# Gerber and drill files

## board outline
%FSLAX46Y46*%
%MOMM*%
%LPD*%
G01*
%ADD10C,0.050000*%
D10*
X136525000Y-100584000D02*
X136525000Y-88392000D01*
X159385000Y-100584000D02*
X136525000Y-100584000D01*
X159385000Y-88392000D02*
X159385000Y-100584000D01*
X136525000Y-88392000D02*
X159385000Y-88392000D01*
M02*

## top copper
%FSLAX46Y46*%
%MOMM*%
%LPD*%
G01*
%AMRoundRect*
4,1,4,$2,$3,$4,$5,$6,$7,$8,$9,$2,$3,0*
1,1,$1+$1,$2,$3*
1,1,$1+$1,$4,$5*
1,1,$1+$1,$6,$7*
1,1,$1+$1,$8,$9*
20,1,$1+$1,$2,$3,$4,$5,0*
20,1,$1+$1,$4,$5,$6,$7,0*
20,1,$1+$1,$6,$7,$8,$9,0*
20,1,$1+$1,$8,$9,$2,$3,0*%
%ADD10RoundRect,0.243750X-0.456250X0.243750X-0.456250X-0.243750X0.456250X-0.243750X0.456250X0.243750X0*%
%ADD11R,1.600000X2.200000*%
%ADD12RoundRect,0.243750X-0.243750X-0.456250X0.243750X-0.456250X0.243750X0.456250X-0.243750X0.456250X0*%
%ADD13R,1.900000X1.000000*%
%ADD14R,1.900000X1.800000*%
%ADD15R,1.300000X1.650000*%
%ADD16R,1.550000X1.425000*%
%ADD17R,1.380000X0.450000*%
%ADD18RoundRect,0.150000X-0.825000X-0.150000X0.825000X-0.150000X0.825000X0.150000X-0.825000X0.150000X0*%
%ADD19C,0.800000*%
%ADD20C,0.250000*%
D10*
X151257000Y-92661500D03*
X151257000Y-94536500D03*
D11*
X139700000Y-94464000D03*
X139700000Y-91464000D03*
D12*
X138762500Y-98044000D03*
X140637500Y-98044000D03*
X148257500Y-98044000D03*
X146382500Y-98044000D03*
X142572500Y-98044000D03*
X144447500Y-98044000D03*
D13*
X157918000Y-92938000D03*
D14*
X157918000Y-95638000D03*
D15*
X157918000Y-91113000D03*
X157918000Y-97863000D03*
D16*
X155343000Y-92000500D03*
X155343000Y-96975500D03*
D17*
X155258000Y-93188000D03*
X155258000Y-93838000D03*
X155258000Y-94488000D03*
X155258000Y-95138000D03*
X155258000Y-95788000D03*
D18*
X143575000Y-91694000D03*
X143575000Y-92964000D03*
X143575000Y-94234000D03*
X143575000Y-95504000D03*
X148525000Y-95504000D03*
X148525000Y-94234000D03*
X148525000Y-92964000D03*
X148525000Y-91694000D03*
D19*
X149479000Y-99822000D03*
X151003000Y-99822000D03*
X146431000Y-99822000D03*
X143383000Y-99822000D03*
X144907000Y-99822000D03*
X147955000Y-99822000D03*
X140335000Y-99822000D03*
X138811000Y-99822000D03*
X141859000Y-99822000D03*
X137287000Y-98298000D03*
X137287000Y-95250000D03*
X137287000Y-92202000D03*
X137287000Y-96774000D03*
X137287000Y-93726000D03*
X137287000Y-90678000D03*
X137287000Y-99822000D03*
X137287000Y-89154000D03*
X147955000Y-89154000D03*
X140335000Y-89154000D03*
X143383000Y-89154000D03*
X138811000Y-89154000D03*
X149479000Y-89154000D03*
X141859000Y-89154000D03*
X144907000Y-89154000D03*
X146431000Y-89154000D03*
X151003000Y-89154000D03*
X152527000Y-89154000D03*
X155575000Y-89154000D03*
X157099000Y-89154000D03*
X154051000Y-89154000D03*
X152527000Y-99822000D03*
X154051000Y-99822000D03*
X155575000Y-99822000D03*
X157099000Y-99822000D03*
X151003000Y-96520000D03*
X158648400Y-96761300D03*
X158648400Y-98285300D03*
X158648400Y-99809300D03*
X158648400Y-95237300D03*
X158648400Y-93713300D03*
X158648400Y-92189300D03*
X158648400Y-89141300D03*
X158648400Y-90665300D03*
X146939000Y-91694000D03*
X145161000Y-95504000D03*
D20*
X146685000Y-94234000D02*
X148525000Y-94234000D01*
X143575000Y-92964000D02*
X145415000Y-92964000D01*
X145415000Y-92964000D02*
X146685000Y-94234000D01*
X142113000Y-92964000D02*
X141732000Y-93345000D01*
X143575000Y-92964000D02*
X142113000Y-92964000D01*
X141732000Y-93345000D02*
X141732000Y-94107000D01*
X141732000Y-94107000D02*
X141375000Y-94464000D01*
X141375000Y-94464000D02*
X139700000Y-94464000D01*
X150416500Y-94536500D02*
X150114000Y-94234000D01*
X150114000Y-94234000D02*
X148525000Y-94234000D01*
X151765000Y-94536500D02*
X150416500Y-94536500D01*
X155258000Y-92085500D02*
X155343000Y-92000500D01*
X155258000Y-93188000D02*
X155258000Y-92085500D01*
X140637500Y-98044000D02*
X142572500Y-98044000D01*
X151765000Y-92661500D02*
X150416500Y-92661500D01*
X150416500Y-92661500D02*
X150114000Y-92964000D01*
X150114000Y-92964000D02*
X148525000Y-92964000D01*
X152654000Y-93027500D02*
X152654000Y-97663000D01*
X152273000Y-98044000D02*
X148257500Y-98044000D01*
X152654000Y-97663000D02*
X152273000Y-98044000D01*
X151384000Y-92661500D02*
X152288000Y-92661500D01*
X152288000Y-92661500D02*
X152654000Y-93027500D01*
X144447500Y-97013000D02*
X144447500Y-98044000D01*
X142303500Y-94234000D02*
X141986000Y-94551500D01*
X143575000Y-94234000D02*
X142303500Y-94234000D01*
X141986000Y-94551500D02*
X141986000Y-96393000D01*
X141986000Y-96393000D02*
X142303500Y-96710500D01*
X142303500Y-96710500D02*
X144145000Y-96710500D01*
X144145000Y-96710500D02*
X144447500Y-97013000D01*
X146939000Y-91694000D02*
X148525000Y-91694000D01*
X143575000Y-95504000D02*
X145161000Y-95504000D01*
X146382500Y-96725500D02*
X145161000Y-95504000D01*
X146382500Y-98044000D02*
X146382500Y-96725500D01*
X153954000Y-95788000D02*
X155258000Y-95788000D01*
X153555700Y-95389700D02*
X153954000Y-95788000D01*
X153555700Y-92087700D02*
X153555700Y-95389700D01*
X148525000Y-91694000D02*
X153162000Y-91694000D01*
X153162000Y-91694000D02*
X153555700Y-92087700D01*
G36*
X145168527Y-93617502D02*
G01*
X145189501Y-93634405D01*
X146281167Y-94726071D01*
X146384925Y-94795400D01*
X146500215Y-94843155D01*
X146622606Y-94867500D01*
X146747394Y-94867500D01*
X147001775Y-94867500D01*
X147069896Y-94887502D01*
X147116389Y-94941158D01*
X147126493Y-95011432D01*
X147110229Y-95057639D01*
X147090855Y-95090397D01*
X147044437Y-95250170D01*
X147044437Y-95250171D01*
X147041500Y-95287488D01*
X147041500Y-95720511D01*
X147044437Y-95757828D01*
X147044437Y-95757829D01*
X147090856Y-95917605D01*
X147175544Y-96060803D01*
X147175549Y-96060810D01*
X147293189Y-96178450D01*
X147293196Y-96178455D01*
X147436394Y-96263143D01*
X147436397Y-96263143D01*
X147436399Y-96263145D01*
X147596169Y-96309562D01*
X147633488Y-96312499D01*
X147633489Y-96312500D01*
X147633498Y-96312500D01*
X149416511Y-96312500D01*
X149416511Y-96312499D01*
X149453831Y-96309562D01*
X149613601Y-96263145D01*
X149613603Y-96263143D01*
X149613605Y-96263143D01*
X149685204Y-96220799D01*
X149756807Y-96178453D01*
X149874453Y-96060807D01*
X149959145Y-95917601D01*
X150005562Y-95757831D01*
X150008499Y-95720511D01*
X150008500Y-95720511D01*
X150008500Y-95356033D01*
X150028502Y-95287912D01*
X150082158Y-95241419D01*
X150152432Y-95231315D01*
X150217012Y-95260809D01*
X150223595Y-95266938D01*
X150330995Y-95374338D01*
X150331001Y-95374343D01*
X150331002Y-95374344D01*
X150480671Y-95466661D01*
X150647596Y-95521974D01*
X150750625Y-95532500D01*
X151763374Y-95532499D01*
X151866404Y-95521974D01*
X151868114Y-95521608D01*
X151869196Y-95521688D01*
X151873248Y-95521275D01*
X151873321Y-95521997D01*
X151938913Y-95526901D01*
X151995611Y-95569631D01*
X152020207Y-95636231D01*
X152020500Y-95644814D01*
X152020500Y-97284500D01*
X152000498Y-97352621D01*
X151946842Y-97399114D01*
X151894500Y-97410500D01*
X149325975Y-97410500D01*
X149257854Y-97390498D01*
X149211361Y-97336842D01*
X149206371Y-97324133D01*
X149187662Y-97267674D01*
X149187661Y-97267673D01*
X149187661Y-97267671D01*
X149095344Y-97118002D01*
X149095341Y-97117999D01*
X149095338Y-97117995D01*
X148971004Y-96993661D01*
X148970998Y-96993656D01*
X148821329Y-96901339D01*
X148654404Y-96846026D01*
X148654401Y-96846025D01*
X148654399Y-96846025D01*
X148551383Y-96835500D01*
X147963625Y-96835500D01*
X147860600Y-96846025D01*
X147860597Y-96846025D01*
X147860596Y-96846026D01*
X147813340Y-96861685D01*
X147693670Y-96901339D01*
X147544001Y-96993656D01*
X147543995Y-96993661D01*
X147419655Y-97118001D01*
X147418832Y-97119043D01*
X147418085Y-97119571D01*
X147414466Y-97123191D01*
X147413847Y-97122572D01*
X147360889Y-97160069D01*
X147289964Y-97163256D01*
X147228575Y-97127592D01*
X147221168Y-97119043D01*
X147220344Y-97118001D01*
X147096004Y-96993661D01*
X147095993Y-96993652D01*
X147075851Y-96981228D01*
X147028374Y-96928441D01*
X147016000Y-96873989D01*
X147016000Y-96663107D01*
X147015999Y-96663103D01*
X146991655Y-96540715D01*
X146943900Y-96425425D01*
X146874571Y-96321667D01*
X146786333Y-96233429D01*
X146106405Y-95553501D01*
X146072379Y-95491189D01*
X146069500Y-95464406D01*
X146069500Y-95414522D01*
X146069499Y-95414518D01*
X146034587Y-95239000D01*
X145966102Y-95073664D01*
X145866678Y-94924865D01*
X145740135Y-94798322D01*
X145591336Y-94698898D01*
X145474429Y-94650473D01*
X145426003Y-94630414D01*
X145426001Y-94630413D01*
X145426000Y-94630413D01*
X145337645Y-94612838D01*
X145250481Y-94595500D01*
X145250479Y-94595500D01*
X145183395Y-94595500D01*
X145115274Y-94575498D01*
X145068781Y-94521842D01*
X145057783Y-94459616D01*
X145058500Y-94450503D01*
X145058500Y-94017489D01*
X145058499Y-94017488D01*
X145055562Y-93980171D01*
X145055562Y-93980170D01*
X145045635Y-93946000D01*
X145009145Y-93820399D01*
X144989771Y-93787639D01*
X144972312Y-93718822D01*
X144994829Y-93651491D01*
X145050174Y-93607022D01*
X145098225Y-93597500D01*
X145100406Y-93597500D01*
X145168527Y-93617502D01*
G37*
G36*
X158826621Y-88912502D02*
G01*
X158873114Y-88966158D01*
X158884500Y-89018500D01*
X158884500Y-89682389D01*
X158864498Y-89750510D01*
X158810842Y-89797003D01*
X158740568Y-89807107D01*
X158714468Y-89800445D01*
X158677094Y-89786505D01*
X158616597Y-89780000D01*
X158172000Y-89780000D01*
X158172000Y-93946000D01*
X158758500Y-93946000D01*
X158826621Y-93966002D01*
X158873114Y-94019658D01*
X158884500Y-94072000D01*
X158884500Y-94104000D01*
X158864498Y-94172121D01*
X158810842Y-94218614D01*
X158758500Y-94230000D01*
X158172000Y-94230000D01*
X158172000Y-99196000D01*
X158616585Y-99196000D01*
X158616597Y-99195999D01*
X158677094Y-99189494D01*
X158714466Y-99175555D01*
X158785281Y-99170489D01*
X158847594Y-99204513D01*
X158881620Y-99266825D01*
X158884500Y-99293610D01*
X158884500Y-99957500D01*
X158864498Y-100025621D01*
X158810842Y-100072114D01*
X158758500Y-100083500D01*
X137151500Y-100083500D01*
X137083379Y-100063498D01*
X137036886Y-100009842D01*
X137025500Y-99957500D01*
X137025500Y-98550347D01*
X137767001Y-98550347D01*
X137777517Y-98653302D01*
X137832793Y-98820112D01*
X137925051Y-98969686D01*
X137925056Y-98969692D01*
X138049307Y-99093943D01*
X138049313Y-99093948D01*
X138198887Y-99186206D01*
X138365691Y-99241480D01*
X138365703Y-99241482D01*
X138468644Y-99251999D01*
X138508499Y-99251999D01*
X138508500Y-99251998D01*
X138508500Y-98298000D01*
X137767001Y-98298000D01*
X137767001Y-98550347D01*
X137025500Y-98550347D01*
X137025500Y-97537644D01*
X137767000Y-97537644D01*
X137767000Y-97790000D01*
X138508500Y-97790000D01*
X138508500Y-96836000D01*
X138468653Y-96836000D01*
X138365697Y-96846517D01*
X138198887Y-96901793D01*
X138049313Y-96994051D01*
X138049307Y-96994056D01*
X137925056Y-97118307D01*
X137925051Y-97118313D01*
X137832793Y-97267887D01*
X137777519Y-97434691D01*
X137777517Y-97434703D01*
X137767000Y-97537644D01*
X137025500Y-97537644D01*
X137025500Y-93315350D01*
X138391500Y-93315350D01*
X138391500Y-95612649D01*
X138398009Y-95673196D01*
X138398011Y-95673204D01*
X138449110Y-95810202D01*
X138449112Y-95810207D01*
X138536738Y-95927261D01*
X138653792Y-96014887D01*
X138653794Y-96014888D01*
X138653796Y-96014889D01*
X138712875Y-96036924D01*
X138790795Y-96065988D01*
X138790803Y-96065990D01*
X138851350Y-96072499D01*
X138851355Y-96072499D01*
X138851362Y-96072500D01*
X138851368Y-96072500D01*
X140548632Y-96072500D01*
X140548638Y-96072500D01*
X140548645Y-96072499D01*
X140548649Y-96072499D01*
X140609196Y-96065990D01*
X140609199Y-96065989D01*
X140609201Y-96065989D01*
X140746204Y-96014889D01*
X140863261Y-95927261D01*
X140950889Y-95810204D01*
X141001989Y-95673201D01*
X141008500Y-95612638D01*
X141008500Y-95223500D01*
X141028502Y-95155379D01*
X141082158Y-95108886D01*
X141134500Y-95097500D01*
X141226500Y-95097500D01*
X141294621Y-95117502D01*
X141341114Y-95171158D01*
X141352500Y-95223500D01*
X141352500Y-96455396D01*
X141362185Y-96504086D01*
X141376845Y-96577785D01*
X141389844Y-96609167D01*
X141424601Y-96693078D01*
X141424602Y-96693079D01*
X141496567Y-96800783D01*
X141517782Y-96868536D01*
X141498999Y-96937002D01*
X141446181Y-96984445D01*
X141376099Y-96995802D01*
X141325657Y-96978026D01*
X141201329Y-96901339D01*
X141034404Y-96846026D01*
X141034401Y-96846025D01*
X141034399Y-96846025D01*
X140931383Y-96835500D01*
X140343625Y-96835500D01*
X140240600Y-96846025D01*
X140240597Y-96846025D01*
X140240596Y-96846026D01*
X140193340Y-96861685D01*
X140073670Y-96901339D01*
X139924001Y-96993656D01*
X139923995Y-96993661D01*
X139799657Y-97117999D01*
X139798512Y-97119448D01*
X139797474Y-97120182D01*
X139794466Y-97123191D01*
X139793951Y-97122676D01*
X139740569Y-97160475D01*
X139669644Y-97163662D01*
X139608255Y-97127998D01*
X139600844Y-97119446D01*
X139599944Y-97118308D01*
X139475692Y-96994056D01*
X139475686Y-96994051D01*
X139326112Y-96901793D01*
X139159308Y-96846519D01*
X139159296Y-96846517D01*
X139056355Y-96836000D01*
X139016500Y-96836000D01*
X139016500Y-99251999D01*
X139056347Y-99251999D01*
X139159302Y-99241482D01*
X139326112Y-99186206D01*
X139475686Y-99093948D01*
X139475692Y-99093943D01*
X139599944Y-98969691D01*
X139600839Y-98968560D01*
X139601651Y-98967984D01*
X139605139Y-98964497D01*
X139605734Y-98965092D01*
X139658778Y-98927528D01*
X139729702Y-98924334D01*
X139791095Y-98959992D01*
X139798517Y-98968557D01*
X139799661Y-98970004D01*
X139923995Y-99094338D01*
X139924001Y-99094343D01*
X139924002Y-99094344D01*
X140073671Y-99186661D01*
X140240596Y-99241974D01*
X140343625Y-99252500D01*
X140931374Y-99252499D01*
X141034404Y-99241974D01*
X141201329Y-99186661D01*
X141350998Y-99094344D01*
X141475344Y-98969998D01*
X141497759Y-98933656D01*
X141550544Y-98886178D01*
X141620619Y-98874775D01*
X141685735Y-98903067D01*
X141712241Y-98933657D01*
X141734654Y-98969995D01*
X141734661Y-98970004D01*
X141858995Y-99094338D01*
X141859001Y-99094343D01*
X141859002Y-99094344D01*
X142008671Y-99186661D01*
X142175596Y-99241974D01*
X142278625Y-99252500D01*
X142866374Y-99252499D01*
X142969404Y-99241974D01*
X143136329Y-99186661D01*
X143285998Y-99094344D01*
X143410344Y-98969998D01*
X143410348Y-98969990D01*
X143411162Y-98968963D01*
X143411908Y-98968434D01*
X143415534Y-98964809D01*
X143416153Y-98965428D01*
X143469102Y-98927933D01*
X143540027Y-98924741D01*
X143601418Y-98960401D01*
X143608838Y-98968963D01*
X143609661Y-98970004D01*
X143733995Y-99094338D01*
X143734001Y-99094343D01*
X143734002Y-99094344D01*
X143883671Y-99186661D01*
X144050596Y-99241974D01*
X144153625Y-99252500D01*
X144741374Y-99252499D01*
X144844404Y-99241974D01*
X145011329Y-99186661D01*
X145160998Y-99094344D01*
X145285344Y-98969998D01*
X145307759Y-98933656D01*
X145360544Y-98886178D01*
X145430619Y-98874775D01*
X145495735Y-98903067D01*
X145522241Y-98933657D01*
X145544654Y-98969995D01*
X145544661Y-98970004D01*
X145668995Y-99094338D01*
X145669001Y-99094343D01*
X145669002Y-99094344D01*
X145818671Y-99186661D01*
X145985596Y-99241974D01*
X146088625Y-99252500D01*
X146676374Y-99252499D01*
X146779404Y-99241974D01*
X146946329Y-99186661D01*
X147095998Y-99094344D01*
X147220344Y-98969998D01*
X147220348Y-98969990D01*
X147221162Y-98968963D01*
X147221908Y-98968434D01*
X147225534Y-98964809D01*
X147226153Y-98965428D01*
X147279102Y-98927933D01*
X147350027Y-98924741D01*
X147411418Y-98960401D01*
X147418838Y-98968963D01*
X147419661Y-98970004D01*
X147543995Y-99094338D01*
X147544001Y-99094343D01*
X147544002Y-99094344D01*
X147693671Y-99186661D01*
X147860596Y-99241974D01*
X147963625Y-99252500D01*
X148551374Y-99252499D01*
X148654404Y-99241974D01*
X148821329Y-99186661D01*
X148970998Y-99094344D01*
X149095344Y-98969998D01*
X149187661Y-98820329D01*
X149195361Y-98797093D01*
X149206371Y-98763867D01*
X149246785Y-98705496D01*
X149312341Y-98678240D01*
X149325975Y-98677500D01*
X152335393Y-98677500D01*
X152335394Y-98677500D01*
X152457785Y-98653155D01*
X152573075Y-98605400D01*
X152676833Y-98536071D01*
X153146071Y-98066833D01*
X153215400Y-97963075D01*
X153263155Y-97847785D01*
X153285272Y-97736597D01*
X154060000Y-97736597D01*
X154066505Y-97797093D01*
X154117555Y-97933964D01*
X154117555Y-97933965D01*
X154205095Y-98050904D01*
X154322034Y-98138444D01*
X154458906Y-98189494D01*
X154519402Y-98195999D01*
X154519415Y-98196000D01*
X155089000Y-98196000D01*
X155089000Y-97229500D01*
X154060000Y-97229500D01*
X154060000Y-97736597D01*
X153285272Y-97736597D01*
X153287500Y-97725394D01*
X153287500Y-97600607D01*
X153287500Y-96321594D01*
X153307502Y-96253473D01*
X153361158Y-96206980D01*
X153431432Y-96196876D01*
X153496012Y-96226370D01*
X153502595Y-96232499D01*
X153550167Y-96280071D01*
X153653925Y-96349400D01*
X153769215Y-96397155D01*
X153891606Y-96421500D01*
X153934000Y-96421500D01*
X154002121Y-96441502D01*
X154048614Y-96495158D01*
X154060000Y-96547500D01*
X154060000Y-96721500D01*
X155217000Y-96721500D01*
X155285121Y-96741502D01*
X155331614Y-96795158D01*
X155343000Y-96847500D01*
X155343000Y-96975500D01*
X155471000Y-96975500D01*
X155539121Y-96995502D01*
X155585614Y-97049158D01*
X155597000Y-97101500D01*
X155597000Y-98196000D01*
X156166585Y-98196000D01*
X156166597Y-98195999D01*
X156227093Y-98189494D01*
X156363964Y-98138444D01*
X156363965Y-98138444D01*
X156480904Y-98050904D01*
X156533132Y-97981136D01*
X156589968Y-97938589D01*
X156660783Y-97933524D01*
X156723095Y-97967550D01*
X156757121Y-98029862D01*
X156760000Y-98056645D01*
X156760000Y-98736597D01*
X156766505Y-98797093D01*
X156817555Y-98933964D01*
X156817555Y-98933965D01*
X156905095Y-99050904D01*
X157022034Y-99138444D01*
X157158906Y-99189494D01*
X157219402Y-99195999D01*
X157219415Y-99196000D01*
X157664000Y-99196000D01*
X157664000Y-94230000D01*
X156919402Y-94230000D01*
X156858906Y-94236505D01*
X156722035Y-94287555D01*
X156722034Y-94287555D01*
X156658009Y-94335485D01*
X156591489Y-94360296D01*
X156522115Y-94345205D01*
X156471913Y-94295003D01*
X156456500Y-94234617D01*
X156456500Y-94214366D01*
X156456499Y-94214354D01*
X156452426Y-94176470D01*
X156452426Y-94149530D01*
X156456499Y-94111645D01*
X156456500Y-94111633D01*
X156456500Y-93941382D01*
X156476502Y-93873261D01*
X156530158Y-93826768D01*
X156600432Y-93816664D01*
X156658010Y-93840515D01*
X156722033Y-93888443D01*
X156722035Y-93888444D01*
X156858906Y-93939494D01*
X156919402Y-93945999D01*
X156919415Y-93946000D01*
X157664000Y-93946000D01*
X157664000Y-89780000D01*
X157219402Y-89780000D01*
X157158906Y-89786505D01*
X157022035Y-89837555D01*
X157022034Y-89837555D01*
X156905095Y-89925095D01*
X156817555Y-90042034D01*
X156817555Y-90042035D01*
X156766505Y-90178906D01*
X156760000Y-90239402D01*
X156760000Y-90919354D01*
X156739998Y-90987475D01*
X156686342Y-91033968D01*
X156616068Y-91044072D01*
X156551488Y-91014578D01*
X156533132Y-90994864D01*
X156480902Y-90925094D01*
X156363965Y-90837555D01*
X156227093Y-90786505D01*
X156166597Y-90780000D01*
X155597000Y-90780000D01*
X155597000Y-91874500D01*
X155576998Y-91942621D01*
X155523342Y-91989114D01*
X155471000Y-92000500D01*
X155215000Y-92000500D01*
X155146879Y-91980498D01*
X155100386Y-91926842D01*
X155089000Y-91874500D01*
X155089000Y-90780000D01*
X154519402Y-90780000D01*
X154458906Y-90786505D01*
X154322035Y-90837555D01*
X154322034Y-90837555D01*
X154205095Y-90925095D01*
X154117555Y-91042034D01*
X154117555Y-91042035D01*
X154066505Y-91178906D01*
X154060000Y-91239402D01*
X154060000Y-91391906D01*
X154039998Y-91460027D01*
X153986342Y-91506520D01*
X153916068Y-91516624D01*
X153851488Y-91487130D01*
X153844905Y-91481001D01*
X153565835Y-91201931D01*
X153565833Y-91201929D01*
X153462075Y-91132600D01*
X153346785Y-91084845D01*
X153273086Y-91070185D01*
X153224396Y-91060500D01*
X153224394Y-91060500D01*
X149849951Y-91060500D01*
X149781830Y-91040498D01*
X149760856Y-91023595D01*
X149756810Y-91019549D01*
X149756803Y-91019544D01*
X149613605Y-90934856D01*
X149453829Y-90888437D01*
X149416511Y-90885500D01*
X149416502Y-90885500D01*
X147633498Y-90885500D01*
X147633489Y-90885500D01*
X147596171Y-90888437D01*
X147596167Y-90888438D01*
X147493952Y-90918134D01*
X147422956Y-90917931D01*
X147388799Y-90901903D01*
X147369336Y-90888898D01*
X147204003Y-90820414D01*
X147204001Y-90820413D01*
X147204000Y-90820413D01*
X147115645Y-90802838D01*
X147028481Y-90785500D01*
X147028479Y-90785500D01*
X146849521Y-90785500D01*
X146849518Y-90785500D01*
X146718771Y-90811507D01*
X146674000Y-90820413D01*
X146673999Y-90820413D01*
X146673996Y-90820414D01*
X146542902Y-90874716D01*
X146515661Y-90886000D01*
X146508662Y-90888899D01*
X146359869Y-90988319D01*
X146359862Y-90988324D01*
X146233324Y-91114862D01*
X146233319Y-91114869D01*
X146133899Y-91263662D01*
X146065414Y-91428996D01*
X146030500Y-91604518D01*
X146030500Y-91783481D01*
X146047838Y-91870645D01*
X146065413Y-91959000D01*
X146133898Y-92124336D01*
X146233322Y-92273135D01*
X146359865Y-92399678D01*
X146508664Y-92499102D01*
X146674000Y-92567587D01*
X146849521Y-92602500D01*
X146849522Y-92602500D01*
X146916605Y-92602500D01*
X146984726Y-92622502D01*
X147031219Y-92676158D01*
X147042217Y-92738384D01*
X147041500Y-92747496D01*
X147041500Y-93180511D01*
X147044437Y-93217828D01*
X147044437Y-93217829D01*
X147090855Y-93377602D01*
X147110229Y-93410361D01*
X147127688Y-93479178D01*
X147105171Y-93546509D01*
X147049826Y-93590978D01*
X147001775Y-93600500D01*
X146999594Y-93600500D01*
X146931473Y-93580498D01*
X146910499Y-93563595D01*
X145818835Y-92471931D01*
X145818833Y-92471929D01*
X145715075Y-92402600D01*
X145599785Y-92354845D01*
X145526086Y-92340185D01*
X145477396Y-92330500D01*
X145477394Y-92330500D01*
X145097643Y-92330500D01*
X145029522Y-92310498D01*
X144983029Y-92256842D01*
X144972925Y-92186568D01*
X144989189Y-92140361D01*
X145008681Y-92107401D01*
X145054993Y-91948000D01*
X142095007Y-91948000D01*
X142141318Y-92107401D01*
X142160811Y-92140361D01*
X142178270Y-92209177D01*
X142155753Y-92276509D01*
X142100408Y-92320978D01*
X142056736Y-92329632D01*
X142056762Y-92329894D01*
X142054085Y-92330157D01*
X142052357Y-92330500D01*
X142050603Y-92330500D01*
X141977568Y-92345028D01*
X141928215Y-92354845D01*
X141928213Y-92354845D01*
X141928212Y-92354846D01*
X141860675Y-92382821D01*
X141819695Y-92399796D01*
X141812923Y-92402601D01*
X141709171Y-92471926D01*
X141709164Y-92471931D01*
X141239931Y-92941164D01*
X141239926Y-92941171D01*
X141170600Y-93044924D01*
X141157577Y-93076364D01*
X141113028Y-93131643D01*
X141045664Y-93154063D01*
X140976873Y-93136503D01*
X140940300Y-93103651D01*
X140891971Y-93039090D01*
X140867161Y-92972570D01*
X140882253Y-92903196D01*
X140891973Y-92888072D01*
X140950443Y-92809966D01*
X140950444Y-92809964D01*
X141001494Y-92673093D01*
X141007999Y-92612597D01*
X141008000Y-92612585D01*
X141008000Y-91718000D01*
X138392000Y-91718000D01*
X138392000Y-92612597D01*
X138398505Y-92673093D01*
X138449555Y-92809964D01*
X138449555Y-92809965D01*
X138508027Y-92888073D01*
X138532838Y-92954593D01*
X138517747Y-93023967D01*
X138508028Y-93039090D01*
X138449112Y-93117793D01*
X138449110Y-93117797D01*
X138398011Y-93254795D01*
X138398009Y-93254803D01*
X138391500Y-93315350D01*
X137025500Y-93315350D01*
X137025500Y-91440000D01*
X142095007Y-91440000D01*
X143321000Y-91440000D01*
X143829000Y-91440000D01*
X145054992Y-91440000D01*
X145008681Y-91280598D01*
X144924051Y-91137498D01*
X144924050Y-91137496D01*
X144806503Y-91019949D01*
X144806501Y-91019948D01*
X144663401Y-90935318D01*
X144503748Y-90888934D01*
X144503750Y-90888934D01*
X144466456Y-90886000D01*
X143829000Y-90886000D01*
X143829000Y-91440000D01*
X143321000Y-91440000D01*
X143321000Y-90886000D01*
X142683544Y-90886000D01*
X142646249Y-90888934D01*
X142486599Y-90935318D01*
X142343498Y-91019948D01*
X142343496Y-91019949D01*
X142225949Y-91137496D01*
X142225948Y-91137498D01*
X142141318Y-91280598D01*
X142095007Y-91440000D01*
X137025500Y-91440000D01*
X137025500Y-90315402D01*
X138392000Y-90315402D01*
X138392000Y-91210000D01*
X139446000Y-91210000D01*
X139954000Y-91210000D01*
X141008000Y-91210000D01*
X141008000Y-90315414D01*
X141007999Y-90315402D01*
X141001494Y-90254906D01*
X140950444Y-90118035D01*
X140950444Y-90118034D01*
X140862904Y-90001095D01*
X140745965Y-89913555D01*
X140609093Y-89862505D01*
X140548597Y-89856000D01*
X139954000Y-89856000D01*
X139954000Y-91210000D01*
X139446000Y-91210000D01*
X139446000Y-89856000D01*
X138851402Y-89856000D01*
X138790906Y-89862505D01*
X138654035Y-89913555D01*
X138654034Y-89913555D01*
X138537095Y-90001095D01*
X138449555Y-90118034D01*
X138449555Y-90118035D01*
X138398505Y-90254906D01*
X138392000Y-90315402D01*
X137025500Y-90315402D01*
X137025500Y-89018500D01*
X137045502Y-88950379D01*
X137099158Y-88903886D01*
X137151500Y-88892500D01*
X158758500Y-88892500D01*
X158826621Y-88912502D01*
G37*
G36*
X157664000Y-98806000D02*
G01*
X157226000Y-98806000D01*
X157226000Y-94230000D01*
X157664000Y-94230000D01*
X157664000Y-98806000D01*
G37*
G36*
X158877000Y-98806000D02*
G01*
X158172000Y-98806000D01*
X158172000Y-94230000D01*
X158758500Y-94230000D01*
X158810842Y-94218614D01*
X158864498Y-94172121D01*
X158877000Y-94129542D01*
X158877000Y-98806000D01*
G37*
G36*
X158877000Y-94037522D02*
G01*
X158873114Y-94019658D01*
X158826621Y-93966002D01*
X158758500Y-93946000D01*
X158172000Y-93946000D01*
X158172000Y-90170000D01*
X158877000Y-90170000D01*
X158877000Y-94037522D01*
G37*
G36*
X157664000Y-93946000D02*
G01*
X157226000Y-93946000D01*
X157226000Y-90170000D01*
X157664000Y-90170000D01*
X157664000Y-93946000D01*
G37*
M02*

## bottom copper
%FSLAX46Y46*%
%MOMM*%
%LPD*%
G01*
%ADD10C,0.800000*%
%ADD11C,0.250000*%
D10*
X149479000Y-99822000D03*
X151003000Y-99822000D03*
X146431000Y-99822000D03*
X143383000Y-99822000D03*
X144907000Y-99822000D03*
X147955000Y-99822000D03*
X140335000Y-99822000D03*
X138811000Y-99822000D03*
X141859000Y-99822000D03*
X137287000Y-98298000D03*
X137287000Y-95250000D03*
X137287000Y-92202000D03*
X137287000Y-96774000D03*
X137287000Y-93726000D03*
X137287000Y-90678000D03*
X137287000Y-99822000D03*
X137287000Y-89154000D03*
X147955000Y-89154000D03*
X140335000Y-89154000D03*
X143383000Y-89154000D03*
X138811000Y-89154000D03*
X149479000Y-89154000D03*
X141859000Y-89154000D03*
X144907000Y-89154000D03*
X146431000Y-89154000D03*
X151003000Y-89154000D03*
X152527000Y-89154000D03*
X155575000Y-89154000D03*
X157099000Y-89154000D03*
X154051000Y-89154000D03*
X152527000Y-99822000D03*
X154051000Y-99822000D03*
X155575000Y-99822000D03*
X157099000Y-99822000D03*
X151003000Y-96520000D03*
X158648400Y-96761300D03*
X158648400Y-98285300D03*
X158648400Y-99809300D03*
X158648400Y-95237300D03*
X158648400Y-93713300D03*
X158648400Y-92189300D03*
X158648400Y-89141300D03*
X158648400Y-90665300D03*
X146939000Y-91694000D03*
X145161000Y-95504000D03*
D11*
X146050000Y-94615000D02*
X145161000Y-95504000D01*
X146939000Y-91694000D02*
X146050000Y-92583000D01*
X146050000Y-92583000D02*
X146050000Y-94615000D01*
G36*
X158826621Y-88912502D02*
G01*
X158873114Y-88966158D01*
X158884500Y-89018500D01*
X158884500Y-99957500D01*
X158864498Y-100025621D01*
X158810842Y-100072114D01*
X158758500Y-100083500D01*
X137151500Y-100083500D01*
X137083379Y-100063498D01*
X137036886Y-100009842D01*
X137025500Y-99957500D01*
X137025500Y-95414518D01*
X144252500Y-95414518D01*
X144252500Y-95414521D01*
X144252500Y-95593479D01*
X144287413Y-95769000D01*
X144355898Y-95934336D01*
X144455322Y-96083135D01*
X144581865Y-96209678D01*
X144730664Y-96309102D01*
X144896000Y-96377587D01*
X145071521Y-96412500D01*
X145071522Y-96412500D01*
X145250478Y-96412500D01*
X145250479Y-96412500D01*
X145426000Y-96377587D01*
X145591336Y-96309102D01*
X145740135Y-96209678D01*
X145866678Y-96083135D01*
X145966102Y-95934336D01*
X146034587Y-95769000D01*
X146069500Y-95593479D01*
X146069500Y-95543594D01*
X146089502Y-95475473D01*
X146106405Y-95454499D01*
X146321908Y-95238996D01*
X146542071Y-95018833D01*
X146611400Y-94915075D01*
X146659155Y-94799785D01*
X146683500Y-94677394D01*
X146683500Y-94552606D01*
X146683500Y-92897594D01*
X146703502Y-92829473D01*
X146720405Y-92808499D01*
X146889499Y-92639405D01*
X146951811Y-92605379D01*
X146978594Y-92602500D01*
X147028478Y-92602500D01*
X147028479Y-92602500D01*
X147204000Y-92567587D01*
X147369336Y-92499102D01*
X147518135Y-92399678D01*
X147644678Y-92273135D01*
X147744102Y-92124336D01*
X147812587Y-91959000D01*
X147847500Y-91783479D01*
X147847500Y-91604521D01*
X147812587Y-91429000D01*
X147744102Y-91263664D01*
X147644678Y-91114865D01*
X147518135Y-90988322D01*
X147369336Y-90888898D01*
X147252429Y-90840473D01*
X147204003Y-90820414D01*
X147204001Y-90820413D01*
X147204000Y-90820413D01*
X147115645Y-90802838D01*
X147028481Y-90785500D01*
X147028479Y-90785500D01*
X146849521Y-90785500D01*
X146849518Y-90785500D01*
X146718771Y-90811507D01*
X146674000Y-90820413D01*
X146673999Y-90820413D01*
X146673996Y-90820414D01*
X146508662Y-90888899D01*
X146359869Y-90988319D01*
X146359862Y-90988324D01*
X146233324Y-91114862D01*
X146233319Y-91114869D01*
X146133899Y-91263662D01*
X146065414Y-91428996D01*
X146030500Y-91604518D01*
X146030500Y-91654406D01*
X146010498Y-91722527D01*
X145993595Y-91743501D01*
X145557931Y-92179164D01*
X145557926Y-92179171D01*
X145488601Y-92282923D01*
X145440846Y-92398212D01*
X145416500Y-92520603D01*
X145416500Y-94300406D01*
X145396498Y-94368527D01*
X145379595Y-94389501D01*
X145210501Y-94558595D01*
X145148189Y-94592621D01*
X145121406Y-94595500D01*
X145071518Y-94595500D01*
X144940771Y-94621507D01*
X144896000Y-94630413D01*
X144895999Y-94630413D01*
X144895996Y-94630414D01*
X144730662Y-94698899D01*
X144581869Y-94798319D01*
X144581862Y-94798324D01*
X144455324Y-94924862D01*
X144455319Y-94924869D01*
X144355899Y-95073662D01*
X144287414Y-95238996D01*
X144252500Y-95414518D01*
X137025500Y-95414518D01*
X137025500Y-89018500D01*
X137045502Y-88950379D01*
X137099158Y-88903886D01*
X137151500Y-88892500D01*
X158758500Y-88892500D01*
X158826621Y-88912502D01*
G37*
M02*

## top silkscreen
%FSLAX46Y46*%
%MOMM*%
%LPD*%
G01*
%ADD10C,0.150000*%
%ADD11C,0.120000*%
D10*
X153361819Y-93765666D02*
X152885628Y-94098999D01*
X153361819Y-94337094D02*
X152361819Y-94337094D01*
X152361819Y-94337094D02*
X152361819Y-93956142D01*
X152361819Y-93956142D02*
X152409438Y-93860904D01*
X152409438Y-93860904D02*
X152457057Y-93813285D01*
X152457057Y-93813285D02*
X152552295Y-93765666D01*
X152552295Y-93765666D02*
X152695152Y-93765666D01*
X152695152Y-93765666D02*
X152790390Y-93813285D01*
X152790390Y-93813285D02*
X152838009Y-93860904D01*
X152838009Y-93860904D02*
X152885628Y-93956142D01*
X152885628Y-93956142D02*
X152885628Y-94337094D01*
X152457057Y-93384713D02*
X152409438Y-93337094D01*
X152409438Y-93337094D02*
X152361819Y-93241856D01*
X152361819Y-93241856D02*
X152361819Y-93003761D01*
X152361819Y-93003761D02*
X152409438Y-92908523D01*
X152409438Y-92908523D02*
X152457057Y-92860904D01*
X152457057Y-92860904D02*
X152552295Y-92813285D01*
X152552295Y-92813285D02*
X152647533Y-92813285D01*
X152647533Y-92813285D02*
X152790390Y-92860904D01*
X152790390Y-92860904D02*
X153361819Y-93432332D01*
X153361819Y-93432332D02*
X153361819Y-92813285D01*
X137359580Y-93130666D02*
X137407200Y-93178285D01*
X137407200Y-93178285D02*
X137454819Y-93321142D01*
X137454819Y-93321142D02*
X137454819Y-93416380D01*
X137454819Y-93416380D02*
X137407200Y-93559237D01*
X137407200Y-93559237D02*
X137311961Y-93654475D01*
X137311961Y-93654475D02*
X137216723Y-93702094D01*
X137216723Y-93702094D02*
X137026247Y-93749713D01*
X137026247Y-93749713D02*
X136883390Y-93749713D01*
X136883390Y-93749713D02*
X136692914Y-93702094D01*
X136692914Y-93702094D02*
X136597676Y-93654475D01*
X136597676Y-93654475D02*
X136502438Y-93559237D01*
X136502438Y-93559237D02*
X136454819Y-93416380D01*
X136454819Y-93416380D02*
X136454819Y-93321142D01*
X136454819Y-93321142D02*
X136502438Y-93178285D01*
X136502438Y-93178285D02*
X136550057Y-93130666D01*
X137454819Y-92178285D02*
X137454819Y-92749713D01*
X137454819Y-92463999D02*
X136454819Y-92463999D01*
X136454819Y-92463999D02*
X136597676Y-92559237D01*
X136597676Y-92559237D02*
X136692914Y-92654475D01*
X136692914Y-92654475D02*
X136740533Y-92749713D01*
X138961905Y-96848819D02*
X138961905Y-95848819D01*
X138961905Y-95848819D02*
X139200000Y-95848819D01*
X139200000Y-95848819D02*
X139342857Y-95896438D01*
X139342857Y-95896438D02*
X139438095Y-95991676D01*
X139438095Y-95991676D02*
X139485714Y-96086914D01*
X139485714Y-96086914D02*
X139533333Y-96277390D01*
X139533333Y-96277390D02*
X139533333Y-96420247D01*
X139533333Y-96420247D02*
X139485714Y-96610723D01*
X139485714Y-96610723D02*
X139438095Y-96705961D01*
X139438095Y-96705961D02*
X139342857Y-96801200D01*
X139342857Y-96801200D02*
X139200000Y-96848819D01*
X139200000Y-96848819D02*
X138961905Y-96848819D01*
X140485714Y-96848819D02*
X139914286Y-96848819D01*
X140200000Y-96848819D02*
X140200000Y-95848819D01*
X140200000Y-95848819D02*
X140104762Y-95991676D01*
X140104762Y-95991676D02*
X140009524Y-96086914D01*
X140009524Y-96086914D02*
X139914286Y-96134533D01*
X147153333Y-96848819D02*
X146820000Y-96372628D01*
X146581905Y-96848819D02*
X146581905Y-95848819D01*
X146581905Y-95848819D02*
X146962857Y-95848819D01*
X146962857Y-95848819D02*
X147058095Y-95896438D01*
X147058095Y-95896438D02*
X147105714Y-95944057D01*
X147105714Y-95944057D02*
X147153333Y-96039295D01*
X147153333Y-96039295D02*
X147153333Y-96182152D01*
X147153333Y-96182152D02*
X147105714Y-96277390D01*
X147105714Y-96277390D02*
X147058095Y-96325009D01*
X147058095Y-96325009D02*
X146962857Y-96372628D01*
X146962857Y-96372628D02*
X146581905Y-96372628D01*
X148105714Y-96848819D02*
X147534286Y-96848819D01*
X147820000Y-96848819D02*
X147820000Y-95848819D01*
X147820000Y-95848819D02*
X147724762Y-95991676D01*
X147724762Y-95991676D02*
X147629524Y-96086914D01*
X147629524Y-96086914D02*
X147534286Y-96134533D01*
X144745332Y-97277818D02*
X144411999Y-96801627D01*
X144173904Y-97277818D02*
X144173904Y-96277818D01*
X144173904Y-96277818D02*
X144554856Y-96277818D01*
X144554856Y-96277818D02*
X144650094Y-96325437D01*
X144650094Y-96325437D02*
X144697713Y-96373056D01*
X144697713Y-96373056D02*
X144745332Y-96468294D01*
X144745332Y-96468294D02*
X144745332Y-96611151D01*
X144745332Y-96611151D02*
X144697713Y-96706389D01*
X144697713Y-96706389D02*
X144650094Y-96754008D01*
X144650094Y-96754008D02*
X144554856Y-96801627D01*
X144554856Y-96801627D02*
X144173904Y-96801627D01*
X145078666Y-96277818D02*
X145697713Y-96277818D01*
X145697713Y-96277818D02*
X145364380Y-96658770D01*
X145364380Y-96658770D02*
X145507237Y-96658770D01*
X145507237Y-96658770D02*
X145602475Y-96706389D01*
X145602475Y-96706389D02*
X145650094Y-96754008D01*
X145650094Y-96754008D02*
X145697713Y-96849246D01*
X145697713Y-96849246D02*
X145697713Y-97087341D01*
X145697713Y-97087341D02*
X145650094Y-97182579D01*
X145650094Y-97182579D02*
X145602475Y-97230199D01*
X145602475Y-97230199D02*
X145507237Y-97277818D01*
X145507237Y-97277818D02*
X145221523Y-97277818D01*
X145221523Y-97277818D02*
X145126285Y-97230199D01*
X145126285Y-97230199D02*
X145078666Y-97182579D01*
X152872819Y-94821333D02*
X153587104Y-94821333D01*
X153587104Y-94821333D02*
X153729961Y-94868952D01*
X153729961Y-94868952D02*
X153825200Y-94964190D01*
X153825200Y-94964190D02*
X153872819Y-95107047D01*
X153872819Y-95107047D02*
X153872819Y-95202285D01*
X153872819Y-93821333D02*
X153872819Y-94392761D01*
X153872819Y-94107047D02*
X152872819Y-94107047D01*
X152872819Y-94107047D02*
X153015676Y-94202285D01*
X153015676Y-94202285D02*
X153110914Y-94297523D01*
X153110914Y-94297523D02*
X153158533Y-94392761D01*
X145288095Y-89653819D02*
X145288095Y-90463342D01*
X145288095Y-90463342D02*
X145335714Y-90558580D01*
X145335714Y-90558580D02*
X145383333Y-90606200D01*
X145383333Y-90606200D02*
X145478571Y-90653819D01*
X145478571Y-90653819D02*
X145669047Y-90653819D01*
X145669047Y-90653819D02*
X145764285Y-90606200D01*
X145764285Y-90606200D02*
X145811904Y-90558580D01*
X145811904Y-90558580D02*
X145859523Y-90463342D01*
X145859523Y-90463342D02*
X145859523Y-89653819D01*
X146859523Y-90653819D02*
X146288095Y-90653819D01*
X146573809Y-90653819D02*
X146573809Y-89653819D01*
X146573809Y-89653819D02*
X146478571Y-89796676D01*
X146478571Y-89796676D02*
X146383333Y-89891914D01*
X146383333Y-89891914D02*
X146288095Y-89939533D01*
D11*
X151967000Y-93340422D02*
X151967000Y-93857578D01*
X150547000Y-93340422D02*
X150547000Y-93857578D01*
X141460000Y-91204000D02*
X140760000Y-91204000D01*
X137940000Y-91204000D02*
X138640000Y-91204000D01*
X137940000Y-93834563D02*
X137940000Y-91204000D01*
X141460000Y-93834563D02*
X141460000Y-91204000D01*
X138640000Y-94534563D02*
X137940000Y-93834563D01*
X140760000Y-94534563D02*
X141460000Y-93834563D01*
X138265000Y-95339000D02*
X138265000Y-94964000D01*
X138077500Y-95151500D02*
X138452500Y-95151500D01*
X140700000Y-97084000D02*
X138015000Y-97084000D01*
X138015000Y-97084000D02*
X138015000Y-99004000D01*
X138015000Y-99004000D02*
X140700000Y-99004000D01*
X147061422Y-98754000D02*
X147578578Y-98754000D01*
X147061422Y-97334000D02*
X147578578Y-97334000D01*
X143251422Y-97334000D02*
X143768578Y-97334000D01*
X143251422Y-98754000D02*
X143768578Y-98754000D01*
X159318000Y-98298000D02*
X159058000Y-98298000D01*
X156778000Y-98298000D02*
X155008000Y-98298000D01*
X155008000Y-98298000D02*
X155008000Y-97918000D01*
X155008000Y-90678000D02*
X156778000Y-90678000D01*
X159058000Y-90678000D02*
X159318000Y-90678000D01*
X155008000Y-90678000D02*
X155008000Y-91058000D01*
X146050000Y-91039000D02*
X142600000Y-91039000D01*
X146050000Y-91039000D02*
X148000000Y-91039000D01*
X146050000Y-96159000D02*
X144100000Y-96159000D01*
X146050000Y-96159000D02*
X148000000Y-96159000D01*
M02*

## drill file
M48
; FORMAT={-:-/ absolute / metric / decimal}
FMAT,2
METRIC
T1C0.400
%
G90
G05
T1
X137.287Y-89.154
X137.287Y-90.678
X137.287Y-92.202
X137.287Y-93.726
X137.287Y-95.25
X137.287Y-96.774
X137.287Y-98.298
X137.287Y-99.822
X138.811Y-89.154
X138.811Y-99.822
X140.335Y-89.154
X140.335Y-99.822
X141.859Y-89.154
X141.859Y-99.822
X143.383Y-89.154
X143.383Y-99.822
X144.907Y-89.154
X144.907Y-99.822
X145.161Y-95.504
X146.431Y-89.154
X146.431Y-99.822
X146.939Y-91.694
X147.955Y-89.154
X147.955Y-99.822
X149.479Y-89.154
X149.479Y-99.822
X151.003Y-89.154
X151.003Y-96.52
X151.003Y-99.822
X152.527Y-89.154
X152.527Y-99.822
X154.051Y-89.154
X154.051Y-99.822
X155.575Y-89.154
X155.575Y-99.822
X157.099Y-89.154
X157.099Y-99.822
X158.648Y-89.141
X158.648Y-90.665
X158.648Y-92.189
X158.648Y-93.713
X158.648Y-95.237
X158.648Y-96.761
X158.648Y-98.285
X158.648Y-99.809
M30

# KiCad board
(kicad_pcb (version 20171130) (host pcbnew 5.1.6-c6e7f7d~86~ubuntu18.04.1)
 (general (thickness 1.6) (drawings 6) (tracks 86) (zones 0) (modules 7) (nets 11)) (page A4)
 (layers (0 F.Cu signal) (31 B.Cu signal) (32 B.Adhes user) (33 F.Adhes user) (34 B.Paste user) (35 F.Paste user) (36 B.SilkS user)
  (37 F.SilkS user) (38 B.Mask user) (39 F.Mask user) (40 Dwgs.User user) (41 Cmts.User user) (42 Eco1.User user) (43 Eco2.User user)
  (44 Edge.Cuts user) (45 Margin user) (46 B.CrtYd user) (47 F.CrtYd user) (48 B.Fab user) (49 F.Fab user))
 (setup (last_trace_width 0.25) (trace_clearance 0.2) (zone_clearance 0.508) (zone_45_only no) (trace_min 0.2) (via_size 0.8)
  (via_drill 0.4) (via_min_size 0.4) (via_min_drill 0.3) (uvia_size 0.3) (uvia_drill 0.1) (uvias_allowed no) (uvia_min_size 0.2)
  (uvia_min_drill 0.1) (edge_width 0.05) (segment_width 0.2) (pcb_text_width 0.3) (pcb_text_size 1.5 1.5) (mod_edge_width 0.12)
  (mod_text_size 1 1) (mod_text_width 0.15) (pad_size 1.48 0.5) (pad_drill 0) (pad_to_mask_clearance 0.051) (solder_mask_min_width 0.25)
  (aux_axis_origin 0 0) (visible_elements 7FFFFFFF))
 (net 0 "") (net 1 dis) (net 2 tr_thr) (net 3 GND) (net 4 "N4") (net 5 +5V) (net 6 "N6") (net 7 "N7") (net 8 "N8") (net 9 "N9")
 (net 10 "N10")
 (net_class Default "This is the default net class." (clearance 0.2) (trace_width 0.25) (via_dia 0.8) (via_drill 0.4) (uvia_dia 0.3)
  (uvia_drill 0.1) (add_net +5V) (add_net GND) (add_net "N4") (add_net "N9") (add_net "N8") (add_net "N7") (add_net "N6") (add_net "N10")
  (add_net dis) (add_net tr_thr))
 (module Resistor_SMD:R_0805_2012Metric (layer F.Cu) (at 151.257 93.599 270)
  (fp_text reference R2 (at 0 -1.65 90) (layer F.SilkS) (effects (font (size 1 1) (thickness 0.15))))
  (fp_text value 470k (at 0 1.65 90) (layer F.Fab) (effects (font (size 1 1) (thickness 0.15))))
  (fp_line (start -0.258578 -0.71) (end 0.258578 -0.71) (layer F.SilkS) (width 0.12))
  (fp_line (start -0.258578 0.71) (end 0.258578 0.71) (layer F.SilkS) (width 0.12))
  (pad 1 smd roundrect (at -0.9375 0 270) (size 0.975 1.4) (layers F.Cu F.Paste F.Mask) (roundrect_rratio 0.25) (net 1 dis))
  (pad 2 smd roundrect (at 0.9375 0 270) (size 0.975 1.4) (layers F.Cu F.Paste F.Mask) (roundrect_rratio 0.25) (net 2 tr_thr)))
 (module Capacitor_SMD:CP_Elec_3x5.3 (layer F.Cu) (at 139.7 92.964 90)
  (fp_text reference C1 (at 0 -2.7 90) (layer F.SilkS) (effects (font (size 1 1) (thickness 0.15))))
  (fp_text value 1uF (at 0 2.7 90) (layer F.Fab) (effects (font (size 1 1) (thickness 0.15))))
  (fp_line (start 1.76 1.76) (end 1.76 1.06) (layer F.SilkS) (width 0.12))
  (fp_line (start 1.76 -1.76) (end 1.76 -1.06) (layer F.SilkS) (width 0.12))
  (fp_line (start -0.870563 -1.76) (end 1.76 -1.76) (layer F.SilkS) (width 0.12))
  (fp_line (start -0.870563 1.76) (end 1.76 1.76) (layer F.SilkS) (width 0.12))
  (fp_line (start -1.570563 -1.06) (end -0.870563 -1.76) (layer F.SilkS) (width 0.12))
  (fp_line (start -1.570563 1.06) (end -0.870563 1.76) (layer F.SilkS) (width 0.12))
  (fp_line (start -2.375 -1.435) (end -2 -1.435) (layer F.SilkS) (width 0.12))
  (fp_line (start -2.1875 -1.6225) (end -2.1875 -1.2475) (layer F.SilkS) (width 0.12))
  (pad 1 smd rect (at -1.5 0 90) (size 2.2 1.6) (layers F.Cu F.Paste F.Mask) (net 2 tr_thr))
  (pad 2 smd rect (at 1.5 0 90) (size 2.2 1.6) (layers F.Cu F.Paste F.Mask) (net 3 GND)))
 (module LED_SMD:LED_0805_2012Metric (layer F.Cu) (at 139.7 98.044)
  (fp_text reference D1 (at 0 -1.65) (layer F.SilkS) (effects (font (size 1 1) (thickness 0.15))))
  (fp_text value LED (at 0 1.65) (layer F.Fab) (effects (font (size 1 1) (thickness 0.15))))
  (fp_line (start 1 -0.96) (end -1.685 -0.96) (layer F.SilkS) (width 0.12))
  (fp_line (start -1.685 -0.96) (end -1.685 0.96) (layer F.SilkS) (width 0.12))
  (fp_line (start -1.685 0.96) (end 1 0.96) (layer F.SilkS) (width 0.12))
  (pad 1 smd roundrect (at -0.9375 0) (size 0.975 1.4) (layers F.Cu F.Paste F.Mask) (roundrect_rratio 0.25) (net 3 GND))
  (pad 2 smd roundrect (at 0.9375 0) (size 0.975 1.4) (layers F.Cu F.Paste F.Mask) (roundrect_rratio 0.25) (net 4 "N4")))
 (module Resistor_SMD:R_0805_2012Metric (layer F.Cu) (at 147.32 98.044)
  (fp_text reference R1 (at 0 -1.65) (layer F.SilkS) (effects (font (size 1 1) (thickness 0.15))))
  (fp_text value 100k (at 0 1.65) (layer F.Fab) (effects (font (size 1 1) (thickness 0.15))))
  (fp_line (start -0.258578 0.71) (end 0.258578 0.71) (layer F.SilkS) (width 0.12))
  (fp_line (start -0.258578 -0.71) (end 0.258578 -0.71) (layer F.SilkS) (width 0.12))
  (pad 2 smd roundrect (at 0.9375 0) (size 0.975 1.4) (layers F.Cu F.Paste F.Mask) (roundrect_rratio 0.25) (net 1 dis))
  (pad 1 smd roundrect (at -0.9375 0) (size 0.975 1.4) (layers F.Cu F.Paste F.Mask) (roundrect_rratio 0.25) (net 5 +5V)))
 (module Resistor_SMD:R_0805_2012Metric (layer F.Cu) (at 143.51 98.044)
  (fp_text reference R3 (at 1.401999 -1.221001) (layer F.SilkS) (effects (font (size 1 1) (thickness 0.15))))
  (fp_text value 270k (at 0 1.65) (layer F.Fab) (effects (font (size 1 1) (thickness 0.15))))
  (fp_line (start -0.258578 -0.71) (end 0.258578 -0.71) (layer F.SilkS) (width 0.12))
  (fp_line (start -0.258578 0.71) (end 0.258578 0.71) (layer F.SilkS) (width 0.12))
  (pad 1 smd roundrect (at -0.9375 0) (size 0.975 1.4) (layers F.Cu F.Paste F.Mask) (roundrect_rratio 0.25) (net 4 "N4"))
  (pad 2 smd roundrect (at 0.9375 0) (size 0.975 1.4) (layers F.Cu F.Paste F.Mask) (roundrect_rratio 0.25) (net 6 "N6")))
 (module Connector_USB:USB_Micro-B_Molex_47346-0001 (layer F.Cu) (at 156.718 94.488 90)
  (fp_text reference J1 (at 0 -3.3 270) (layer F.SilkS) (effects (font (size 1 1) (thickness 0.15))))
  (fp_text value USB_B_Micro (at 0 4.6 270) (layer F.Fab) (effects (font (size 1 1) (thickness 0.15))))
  (fp_line (start -3.81 2.6) (end -3.81 2.34) (layer F.SilkS) (width 0.12))
  (fp_line (start -3.81 0.06) (end -3.81 -1.71) (layer F.SilkS) (width 0.12))
  (fp_line (start -3.81 -1.71) (end -3.43 -1.71) (layer F.SilkS) (width 0.12))
  (fp_line (start 3.81 -1.71) (end 3.81 0.06) (layer F.SilkS) (width 0.12))
  (fp_line (start 3.81 2.34) (end 3.81 2.6) (layer F.SilkS) (width 0.12))
  (fp_line (start 3.81 -1.71) (end 3.43 -1.71) (layer F.SilkS) (width 0.12))
  (pad 6 smd rect (at 1.55 1.2 90) (size 1 1.9) (layers F.Cu F.Paste F.Mask) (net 3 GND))
  (pad 6 smd rect (at -1.15 1.2 90) (size 1.8 1.9) (layers F.Cu F.Paste F.Mask) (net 3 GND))
  (pad 6 smd rect (at 3.375 1.2 90) (size 1.65 1.3) (layers F.Cu F.Paste F.Mask) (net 3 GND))
  (pad 6 smd rect (at -3.375 1.2 90) (size 1.65 1.3) (layers F.Cu F.Paste F.Mask) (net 3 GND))
  (pad 6 smd rect (at 2.4875 -1.375 90) (size 1.425 1.55) (layers F.Cu F.Paste F.Mask) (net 3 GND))
  (pad 6 smd rect (at -2.4875 -1.375 90) (size 1.425 1.55) (layers F.Cu F.Paste F.Mask) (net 3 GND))
  (pad 5 smd rect (at 1.3 -1.46 90) (size 0.45 1.38) (layers F.Cu F.Paste F.Mask) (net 3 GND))
  (pad 4 smd rect (at 0.65 -1.46 90) (size 0.45 1.38) (layers F.Cu F.Paste F.Mask) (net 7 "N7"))
  (pad 3 smd rect (at 0 -1.46 90) (size 0.45 1.38) (layers F.Cu F.Paste F.Mask) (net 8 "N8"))
  (pad 2 smd rect (at -0.65 -1.46 90) (size 0.45 1.38) (layers F.Cu F.Paste F.Mask) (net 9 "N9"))
  (pad 1 smd rect (at -1.3 -1.46 90) (size 0.45 1.38) (layers F.Cu F.Paste F.Mask) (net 5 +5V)))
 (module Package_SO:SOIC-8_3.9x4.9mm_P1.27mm (layer F.Cu) (at 146.05 93.599)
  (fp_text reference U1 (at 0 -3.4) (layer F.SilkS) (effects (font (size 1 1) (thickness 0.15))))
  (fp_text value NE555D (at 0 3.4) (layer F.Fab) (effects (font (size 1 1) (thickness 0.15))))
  (fp_line (start 0 -2.56) (end -3.45 -2.56) (layer F.SilkS) (width 0.12))
  (fp_line (start 0 -2.56) (end 1.95 -2.56) (layer F.SilkS) (width 0.12))
  (fp_line (start 0 2.56) (end -1.95 2.56) (layer F.SilkS) (width 0.12))
  (fp_line (start 0 2.56) (end 1.95 2.56) (layer F.SilkS) (width 0.12))
  (pad 1 smd roundrect (at -2.475 -1.905) (size 1.95 0.6) (layers F.Cu F.Paste F.Mask) (roundrect_rratio 0.25) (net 3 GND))
  (pad 2 smd roundrect (at -2.475 -0.635) (size 1.95 0.6) (layers F.Cu F.Paste F.Mask) (roundrect_rratio 0.25) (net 2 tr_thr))
  (pad 3 smd roundrect (at -2.475 0.635) (size 1.95 0.6) (layers F.Cu F.Paste F.Mask) (roundrect_rratio 0.25) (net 6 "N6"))
  (pad 4 smd roundrect (at -2.475 1.905) (size 1.95 0.6) (layers F.Cu F.Paste F.Mask) (roundrect_rratio 0.25) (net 5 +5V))
  (pad 5 smd roundrect (at 2.475 1.905) (size 1.95 0.6) (layers F.Cu F.Paste F.Mask) (roundrect_rratio 0.25) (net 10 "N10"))
  (pad 6 smd roundrect (at 2.475 0.635) (size 1.95 0.6) (layers F.Cu F.Paste F.Mask) (roundrect_rratio 0.25) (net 2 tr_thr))
  (pad 7 smd roundrect (at 2.475 -0.635) (size 1.95 0.6) (layers F.Cu F.Paste F.Mask) (roundrect_rratio 0.25) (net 1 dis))
  (pad 8 smd roundrect (at 2.475 -1.905) (size 1.95 0.6) (layers F.Cu F.Paste F.Mask) (roundrect_rratio 0.25) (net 5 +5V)))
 (gr_line (start 136.525 100.584) (end 136.525 88.392) (layer Edge.Cuts) (width 0.05))
 (gr_line (start 159.385 100.584) (end 136.525 100.584) (layer Edge.Cuts) (width 0.05))
 (gr_line (start 159.385 88.392) (end 159.385 100.584) (layer Edge.Cuts) (width 0.05))
 (gr_line (start 136.525 88.392) (end 159.385 88.392) (layer Edge.Cuts) (width 0.05))
 (segment (start 146.685 94.234) (end 148.525 94.234) (width 0.25) (layer F.Cu) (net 2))
 (segment (start 143.575 92.964) (end 145.415 92.964) (width 0.25) (layer F.Cu) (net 2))
 (segment (start 145.415 92.964) (end 146.685 94.234) (width 0.25) (layer F.Cu) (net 2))
 (segment (start 142.113 92.964) (end 141.732 93.345) (width 0.25) (layer F.Cu) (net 2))
 (segment (start 143.575 92.964) (end 142.113 92.964) (width 0.25) (layer F.Cu) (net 2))
 (segment (start 141.732 93.345) (end 141.732 94.107) (width 0.25) (layer F.Cu) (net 2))
 (segment (start 141.732 94.107) (end 141.375 94.464) (width 0.25) (layer F.Cu) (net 2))
 (segment (start 141.375 94.464) (end 139.7 94.464) (width 0.25) (layer F.Cu) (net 2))
 (segment (start 150.4165 94.5365) (end 150.114 94.234) (width 0.25) (layer F.Cu) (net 2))
 (segment (start 150.114 94.234) (end 148.525 94.234) (width 0.25) (layer F.Cu) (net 2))
 (segment (start 151.765 94.5365) (end 150.4165 94.5365) (width 0.25) (layer F.Cu) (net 2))
 (via (at 149.479 99.822) (size 0.8) (drill 0.4) (layers F.Cu B.Cu) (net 3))
 (via (at 151.003 99.822) (size 0.8) (drill 0.4) (layers F.Cu B.Cu) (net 3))
 (via (at 146.431 99.822) (size 0.8) (drill 0.4) (layers F.Cu B.Cu) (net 3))
 (via (at 143.383 99.822) (size 0.8) (drill 0.4) (layers F.Cu B.Cu) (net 3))
 (via (at 144.907 99.822) (size 0.8) (drill 0.4) (layers F.Cu B.Cu) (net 3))
 (via (at 147.955 99.822) (size 0.8) (drill 0.4) (layers F.Cu B.Cu) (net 3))
 (via (at 140.335 99.822) (size 0.8) (drill 0.4) (layers F.Cu B.Cu) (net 3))
 (via (at 138.811 99.822) (size 0.8) (drill 0.4) (layers F.Cu B.Cu) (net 3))
 (via (at 141.859 99.822) (size 0.8) (drill 0.4) (layers F.Cu B.Cu) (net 3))
 (via (at 137.287 98.298) (size 0.8) (drill 0.4) (layers F.Cu B.Cu) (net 3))
 (via (at 137.287 95.25) (size 0.8) (drill 0.4) (layers F.Cu B.Cu) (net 3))
 (via (at 137.287 92.202) (size 0.8) (drill 0.4) (layers F.Cu B.Cu) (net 3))
 (via (at 137.287 96.774) (size 0.8) (drill 0.4) (layers F.Cu B.Cu) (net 3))
 (via (at 137.287 93.726) (size 0.8) (drill 0.4) (layers F.Cu B.Cu) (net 3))
 (via (at 137.287 90.678) (size 0.8) (drill 0.4) (layers F.Cu B.Cu) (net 3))
 (via (at 137.287 99.822) (size 0.8) (drill 0.4) (layers F.Cu B.Cu) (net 3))
 (via (at 137.287 89.154) (size 0.8) (drill 0.4) (layers F.Cu B.Cu) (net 3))
 (via (at 147.955 89.154) (size 0.8) (drill 0.4) (layers F.Cu B.Cu) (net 3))
 (via (at 140.335 89.154) (size 0.8) (drill 0.4) (layers F.Cu B.Cu) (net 3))
 (via (at 143.383 89.154) (size 0.8) (drill 0.4) (layers F.Cu B.Cu) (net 3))
 (via (at 138.811 89.154) (size 0.8) (drill 0.4) (layers F.Cu B.Cu) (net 3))
 (via (at 149.479 89.154) (size 0.8) (drill 0.4) (layers F.Cu B.Cu) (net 3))
 (via (at 141.859 89.154) (size 0.8) (drill 0.4) (layers F.Cu B.Cu) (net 3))
 (via (at 144.907 89.154) (size 0.8) (drill 0.4) (layers F.Cu B.Cu) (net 3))
 (via (at 146.431 89.154) (size 0.8) (drill 0.4) (layers F.Cu B.Cu) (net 3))
 (via (at 151.003 89.154) (size 0.8) (drill 0.4) (layers F.Cu B.Cu) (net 3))
 (via (at 152.527 89.154) (size 0.8) (drill 0.4) (layers F.Cu B.Cu) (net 3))
 (via (at 155.575 89.154) (size 0.8) (drill 0.4) (layers F.Cu B.Cu) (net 3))
 (via (at 157.099 89.154) (size 0.8) (drill 0.4) (layers F.Cu B.Cu) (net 3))
 (via (at 154.051 89.154) (size 0.8) (drill 0.4) (layers F.Cu B.Cu) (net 3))
 (via (at 152.527 99.822) (size 0.8) (drill 0.4) (layers F.Cu B.Cu) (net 3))
 (via (at 154.051 99.822) (size 0.8) (drill 0.4) (layers F.Cu B.Cu) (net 3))
 (via (at 155.575 99.822) (size 0.8) (drill 0.4) (layers F.Cu B.Cu) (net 3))
 (via (at 157.099 99.822) (size 0.8) (drill 0.4) (layers F.Cu B.Cu) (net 3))
 (via (at 151.003 96.52) (size 0.8) (drill 0.4) (layers F.Cu B.Cu) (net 3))
 (via (at 158.6484 96.7613) (size 0.8) (drill 0.4) (layers F.Cu B.Cu) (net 3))
 (via (at 158.6484 98.2853) (size 0.8) (drill 0.4) (layers F.Cu B.Cu) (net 3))
 (via (at 158.6484 99.8093) (size 0.8) (drill 0.4) (layers F.Cu B.Cu) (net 3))
 (via (at 158.6484 95.2373) (size 0.8) (drill 0.4) (layers F.Cu B.Cu) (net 3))
 (via (at 158.6484 93.7133) (size 0.8) (drill 0.4) (layers F.Cu B.Cu) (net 3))
 (via (at 158.6484 92.1893) (size 0.8) (drill 0.4) (layers F.Cu B.Cu) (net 3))
 (via (at 158.6484 89.1413) (size 0.8) (drill 0.4) (layers F.Cu B.Cu) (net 3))
 (via (at 158.6484 90.6653) (size 0.8) (drill 0.4) (layers F.Cu B.Cu) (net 3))
 (segment (start 155.258 92.0855) (end 155.343 92.0005) (width 0.25) (layer F.Cu) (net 3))
 (segment (start 155.258 93.188) (end 155.258 92.0855) (width 0.25) (layer F.Cu) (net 3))
 (segment (start 140.6375 98.044) (end 142.5725 98.044) (width 0.25) (layer F.Cu) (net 4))
 (segment (start 151.765 92.6615) (end 150.4165 92.6615) (width 0.25) (layer F.Cu) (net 1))
 (segment (start 150.4165 92.6615) (end 150.114 92.964) (width 0.25) (layer F.Cu) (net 1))
 (segment (start 150.114 92.964) (end 148.525 92.964) (width 0.25) (layer F.Cu) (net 1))
 (segment (start 152.654 93.0275) (end 152.654 97.663) (width 0.25) (layer F.Cu) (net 1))
 (segment (start 152.273 98.044) (end 148.2575 98.044) (width 0.25) (layer F.Cu) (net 1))
 (segment (start 152.654 97.663) (end 152.273 98.044) (width 0.25) (layer F.Cu) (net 1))
 (segment (start 151.384 92.6615) (end 152.288 92.6615) (width 0.25) (layer F.Cu) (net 1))
 (segment (start 152.288 92.6615) (end 152.654 93.0275) (width 0.25) (layer F.Cu) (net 1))
 (segment (start 144.4475 97.013) (end 144.4475 98.044) (width 0.25) (layer F.Cu) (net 6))
 (segment (start 142.3035 94.234) (end 141.986 94.5515) (width 0.25) (layer F.Cu) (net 6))
 (segment (start 143.575 94.234) (end 142.3035 94.234) (width 0.25) (layer F.Cu) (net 6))
 (segment (start 141.986 94.5515) (end 141.986 96.393) (width 0.25) (layer F.Cu) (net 6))
 (segment (start 141.986 96.393) (end 142.3035 96.7105) (width 0.25) (layer F.Cu) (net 6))
 (segment (start 142.3035 96.7105) (end 144.145 96.7105) (width 0.25) (layer F.Cu) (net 6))
 (segment (start 144.145 96.7105) (end 144.4475 97.013) (width 0.25) (layer F.Cu) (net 6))
 (via (at 146.939 91.694) (size 0.8) (drill 0.4) (layers F.Cu B.Cu) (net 5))
 (via (at 145.161 95.504) (size 0.8) (drill 0.4) (layers F.Cu B.Cu) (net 5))
 (segment (start 146.939 91.694) (end 148.525 91.694) (width 0.25) (layer F.Cu) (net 5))
 (segment (start 143.575 95.504) (end 145.161 95.504) (width 0.25) (layer F.Cu) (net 5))
 (segment (start 146.3825 96.7255) (end 145.161 95.504) (width 0.25) (layer F.Cu) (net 5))
 (segment (start 146.3825 98.044) (end 146.3825 96.7255) (width 0.25) (layer F.Cu) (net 5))
 (segment (start 146.05 94.615) (end 145.161 95.504) (width 0.25) (layer B.Cu) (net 5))
 (segment (start 146.939 91.694) (end 146.05 92.583) (width 0.25) (layer B.Cu) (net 5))
 (segment (start 146.05 92.583) (end 146.05 94.615) (width 0.25) (layer B.Cu) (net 5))
 (segment (start 153.954 95.788) (end 155.258 95.788) (width 0.25) (layer F.Cu) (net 5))
 (segment (start 153.5557 95.3897) (end 153.954 95.788) (width 0.25) (layer F.Cu) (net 5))
 (segment (start 153.5557 92.0877) (end 153.5557 95.3897) (width 0.25) (layer F.Cu) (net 5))
 (segment (start 148.525 91.694) (end 153.162 91.694) (width 0.25) (layer F.Cu) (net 5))
 (segment (start 153.162 91.694) (end 153.5557 92.0877) (width 0.25) (layer F.Cu) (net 5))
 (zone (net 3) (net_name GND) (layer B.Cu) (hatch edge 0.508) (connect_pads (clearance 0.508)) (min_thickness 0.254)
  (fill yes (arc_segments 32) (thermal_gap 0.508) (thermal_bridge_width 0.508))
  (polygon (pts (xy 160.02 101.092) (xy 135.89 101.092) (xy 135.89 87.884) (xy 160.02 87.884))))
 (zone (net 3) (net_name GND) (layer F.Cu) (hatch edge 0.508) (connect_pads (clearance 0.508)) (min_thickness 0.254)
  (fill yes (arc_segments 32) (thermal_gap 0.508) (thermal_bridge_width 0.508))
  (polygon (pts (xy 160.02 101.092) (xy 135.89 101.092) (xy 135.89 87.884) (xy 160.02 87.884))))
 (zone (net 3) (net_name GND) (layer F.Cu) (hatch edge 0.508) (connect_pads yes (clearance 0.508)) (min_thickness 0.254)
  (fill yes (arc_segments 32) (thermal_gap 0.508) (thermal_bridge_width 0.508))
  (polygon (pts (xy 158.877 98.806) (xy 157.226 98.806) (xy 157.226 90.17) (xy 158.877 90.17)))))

